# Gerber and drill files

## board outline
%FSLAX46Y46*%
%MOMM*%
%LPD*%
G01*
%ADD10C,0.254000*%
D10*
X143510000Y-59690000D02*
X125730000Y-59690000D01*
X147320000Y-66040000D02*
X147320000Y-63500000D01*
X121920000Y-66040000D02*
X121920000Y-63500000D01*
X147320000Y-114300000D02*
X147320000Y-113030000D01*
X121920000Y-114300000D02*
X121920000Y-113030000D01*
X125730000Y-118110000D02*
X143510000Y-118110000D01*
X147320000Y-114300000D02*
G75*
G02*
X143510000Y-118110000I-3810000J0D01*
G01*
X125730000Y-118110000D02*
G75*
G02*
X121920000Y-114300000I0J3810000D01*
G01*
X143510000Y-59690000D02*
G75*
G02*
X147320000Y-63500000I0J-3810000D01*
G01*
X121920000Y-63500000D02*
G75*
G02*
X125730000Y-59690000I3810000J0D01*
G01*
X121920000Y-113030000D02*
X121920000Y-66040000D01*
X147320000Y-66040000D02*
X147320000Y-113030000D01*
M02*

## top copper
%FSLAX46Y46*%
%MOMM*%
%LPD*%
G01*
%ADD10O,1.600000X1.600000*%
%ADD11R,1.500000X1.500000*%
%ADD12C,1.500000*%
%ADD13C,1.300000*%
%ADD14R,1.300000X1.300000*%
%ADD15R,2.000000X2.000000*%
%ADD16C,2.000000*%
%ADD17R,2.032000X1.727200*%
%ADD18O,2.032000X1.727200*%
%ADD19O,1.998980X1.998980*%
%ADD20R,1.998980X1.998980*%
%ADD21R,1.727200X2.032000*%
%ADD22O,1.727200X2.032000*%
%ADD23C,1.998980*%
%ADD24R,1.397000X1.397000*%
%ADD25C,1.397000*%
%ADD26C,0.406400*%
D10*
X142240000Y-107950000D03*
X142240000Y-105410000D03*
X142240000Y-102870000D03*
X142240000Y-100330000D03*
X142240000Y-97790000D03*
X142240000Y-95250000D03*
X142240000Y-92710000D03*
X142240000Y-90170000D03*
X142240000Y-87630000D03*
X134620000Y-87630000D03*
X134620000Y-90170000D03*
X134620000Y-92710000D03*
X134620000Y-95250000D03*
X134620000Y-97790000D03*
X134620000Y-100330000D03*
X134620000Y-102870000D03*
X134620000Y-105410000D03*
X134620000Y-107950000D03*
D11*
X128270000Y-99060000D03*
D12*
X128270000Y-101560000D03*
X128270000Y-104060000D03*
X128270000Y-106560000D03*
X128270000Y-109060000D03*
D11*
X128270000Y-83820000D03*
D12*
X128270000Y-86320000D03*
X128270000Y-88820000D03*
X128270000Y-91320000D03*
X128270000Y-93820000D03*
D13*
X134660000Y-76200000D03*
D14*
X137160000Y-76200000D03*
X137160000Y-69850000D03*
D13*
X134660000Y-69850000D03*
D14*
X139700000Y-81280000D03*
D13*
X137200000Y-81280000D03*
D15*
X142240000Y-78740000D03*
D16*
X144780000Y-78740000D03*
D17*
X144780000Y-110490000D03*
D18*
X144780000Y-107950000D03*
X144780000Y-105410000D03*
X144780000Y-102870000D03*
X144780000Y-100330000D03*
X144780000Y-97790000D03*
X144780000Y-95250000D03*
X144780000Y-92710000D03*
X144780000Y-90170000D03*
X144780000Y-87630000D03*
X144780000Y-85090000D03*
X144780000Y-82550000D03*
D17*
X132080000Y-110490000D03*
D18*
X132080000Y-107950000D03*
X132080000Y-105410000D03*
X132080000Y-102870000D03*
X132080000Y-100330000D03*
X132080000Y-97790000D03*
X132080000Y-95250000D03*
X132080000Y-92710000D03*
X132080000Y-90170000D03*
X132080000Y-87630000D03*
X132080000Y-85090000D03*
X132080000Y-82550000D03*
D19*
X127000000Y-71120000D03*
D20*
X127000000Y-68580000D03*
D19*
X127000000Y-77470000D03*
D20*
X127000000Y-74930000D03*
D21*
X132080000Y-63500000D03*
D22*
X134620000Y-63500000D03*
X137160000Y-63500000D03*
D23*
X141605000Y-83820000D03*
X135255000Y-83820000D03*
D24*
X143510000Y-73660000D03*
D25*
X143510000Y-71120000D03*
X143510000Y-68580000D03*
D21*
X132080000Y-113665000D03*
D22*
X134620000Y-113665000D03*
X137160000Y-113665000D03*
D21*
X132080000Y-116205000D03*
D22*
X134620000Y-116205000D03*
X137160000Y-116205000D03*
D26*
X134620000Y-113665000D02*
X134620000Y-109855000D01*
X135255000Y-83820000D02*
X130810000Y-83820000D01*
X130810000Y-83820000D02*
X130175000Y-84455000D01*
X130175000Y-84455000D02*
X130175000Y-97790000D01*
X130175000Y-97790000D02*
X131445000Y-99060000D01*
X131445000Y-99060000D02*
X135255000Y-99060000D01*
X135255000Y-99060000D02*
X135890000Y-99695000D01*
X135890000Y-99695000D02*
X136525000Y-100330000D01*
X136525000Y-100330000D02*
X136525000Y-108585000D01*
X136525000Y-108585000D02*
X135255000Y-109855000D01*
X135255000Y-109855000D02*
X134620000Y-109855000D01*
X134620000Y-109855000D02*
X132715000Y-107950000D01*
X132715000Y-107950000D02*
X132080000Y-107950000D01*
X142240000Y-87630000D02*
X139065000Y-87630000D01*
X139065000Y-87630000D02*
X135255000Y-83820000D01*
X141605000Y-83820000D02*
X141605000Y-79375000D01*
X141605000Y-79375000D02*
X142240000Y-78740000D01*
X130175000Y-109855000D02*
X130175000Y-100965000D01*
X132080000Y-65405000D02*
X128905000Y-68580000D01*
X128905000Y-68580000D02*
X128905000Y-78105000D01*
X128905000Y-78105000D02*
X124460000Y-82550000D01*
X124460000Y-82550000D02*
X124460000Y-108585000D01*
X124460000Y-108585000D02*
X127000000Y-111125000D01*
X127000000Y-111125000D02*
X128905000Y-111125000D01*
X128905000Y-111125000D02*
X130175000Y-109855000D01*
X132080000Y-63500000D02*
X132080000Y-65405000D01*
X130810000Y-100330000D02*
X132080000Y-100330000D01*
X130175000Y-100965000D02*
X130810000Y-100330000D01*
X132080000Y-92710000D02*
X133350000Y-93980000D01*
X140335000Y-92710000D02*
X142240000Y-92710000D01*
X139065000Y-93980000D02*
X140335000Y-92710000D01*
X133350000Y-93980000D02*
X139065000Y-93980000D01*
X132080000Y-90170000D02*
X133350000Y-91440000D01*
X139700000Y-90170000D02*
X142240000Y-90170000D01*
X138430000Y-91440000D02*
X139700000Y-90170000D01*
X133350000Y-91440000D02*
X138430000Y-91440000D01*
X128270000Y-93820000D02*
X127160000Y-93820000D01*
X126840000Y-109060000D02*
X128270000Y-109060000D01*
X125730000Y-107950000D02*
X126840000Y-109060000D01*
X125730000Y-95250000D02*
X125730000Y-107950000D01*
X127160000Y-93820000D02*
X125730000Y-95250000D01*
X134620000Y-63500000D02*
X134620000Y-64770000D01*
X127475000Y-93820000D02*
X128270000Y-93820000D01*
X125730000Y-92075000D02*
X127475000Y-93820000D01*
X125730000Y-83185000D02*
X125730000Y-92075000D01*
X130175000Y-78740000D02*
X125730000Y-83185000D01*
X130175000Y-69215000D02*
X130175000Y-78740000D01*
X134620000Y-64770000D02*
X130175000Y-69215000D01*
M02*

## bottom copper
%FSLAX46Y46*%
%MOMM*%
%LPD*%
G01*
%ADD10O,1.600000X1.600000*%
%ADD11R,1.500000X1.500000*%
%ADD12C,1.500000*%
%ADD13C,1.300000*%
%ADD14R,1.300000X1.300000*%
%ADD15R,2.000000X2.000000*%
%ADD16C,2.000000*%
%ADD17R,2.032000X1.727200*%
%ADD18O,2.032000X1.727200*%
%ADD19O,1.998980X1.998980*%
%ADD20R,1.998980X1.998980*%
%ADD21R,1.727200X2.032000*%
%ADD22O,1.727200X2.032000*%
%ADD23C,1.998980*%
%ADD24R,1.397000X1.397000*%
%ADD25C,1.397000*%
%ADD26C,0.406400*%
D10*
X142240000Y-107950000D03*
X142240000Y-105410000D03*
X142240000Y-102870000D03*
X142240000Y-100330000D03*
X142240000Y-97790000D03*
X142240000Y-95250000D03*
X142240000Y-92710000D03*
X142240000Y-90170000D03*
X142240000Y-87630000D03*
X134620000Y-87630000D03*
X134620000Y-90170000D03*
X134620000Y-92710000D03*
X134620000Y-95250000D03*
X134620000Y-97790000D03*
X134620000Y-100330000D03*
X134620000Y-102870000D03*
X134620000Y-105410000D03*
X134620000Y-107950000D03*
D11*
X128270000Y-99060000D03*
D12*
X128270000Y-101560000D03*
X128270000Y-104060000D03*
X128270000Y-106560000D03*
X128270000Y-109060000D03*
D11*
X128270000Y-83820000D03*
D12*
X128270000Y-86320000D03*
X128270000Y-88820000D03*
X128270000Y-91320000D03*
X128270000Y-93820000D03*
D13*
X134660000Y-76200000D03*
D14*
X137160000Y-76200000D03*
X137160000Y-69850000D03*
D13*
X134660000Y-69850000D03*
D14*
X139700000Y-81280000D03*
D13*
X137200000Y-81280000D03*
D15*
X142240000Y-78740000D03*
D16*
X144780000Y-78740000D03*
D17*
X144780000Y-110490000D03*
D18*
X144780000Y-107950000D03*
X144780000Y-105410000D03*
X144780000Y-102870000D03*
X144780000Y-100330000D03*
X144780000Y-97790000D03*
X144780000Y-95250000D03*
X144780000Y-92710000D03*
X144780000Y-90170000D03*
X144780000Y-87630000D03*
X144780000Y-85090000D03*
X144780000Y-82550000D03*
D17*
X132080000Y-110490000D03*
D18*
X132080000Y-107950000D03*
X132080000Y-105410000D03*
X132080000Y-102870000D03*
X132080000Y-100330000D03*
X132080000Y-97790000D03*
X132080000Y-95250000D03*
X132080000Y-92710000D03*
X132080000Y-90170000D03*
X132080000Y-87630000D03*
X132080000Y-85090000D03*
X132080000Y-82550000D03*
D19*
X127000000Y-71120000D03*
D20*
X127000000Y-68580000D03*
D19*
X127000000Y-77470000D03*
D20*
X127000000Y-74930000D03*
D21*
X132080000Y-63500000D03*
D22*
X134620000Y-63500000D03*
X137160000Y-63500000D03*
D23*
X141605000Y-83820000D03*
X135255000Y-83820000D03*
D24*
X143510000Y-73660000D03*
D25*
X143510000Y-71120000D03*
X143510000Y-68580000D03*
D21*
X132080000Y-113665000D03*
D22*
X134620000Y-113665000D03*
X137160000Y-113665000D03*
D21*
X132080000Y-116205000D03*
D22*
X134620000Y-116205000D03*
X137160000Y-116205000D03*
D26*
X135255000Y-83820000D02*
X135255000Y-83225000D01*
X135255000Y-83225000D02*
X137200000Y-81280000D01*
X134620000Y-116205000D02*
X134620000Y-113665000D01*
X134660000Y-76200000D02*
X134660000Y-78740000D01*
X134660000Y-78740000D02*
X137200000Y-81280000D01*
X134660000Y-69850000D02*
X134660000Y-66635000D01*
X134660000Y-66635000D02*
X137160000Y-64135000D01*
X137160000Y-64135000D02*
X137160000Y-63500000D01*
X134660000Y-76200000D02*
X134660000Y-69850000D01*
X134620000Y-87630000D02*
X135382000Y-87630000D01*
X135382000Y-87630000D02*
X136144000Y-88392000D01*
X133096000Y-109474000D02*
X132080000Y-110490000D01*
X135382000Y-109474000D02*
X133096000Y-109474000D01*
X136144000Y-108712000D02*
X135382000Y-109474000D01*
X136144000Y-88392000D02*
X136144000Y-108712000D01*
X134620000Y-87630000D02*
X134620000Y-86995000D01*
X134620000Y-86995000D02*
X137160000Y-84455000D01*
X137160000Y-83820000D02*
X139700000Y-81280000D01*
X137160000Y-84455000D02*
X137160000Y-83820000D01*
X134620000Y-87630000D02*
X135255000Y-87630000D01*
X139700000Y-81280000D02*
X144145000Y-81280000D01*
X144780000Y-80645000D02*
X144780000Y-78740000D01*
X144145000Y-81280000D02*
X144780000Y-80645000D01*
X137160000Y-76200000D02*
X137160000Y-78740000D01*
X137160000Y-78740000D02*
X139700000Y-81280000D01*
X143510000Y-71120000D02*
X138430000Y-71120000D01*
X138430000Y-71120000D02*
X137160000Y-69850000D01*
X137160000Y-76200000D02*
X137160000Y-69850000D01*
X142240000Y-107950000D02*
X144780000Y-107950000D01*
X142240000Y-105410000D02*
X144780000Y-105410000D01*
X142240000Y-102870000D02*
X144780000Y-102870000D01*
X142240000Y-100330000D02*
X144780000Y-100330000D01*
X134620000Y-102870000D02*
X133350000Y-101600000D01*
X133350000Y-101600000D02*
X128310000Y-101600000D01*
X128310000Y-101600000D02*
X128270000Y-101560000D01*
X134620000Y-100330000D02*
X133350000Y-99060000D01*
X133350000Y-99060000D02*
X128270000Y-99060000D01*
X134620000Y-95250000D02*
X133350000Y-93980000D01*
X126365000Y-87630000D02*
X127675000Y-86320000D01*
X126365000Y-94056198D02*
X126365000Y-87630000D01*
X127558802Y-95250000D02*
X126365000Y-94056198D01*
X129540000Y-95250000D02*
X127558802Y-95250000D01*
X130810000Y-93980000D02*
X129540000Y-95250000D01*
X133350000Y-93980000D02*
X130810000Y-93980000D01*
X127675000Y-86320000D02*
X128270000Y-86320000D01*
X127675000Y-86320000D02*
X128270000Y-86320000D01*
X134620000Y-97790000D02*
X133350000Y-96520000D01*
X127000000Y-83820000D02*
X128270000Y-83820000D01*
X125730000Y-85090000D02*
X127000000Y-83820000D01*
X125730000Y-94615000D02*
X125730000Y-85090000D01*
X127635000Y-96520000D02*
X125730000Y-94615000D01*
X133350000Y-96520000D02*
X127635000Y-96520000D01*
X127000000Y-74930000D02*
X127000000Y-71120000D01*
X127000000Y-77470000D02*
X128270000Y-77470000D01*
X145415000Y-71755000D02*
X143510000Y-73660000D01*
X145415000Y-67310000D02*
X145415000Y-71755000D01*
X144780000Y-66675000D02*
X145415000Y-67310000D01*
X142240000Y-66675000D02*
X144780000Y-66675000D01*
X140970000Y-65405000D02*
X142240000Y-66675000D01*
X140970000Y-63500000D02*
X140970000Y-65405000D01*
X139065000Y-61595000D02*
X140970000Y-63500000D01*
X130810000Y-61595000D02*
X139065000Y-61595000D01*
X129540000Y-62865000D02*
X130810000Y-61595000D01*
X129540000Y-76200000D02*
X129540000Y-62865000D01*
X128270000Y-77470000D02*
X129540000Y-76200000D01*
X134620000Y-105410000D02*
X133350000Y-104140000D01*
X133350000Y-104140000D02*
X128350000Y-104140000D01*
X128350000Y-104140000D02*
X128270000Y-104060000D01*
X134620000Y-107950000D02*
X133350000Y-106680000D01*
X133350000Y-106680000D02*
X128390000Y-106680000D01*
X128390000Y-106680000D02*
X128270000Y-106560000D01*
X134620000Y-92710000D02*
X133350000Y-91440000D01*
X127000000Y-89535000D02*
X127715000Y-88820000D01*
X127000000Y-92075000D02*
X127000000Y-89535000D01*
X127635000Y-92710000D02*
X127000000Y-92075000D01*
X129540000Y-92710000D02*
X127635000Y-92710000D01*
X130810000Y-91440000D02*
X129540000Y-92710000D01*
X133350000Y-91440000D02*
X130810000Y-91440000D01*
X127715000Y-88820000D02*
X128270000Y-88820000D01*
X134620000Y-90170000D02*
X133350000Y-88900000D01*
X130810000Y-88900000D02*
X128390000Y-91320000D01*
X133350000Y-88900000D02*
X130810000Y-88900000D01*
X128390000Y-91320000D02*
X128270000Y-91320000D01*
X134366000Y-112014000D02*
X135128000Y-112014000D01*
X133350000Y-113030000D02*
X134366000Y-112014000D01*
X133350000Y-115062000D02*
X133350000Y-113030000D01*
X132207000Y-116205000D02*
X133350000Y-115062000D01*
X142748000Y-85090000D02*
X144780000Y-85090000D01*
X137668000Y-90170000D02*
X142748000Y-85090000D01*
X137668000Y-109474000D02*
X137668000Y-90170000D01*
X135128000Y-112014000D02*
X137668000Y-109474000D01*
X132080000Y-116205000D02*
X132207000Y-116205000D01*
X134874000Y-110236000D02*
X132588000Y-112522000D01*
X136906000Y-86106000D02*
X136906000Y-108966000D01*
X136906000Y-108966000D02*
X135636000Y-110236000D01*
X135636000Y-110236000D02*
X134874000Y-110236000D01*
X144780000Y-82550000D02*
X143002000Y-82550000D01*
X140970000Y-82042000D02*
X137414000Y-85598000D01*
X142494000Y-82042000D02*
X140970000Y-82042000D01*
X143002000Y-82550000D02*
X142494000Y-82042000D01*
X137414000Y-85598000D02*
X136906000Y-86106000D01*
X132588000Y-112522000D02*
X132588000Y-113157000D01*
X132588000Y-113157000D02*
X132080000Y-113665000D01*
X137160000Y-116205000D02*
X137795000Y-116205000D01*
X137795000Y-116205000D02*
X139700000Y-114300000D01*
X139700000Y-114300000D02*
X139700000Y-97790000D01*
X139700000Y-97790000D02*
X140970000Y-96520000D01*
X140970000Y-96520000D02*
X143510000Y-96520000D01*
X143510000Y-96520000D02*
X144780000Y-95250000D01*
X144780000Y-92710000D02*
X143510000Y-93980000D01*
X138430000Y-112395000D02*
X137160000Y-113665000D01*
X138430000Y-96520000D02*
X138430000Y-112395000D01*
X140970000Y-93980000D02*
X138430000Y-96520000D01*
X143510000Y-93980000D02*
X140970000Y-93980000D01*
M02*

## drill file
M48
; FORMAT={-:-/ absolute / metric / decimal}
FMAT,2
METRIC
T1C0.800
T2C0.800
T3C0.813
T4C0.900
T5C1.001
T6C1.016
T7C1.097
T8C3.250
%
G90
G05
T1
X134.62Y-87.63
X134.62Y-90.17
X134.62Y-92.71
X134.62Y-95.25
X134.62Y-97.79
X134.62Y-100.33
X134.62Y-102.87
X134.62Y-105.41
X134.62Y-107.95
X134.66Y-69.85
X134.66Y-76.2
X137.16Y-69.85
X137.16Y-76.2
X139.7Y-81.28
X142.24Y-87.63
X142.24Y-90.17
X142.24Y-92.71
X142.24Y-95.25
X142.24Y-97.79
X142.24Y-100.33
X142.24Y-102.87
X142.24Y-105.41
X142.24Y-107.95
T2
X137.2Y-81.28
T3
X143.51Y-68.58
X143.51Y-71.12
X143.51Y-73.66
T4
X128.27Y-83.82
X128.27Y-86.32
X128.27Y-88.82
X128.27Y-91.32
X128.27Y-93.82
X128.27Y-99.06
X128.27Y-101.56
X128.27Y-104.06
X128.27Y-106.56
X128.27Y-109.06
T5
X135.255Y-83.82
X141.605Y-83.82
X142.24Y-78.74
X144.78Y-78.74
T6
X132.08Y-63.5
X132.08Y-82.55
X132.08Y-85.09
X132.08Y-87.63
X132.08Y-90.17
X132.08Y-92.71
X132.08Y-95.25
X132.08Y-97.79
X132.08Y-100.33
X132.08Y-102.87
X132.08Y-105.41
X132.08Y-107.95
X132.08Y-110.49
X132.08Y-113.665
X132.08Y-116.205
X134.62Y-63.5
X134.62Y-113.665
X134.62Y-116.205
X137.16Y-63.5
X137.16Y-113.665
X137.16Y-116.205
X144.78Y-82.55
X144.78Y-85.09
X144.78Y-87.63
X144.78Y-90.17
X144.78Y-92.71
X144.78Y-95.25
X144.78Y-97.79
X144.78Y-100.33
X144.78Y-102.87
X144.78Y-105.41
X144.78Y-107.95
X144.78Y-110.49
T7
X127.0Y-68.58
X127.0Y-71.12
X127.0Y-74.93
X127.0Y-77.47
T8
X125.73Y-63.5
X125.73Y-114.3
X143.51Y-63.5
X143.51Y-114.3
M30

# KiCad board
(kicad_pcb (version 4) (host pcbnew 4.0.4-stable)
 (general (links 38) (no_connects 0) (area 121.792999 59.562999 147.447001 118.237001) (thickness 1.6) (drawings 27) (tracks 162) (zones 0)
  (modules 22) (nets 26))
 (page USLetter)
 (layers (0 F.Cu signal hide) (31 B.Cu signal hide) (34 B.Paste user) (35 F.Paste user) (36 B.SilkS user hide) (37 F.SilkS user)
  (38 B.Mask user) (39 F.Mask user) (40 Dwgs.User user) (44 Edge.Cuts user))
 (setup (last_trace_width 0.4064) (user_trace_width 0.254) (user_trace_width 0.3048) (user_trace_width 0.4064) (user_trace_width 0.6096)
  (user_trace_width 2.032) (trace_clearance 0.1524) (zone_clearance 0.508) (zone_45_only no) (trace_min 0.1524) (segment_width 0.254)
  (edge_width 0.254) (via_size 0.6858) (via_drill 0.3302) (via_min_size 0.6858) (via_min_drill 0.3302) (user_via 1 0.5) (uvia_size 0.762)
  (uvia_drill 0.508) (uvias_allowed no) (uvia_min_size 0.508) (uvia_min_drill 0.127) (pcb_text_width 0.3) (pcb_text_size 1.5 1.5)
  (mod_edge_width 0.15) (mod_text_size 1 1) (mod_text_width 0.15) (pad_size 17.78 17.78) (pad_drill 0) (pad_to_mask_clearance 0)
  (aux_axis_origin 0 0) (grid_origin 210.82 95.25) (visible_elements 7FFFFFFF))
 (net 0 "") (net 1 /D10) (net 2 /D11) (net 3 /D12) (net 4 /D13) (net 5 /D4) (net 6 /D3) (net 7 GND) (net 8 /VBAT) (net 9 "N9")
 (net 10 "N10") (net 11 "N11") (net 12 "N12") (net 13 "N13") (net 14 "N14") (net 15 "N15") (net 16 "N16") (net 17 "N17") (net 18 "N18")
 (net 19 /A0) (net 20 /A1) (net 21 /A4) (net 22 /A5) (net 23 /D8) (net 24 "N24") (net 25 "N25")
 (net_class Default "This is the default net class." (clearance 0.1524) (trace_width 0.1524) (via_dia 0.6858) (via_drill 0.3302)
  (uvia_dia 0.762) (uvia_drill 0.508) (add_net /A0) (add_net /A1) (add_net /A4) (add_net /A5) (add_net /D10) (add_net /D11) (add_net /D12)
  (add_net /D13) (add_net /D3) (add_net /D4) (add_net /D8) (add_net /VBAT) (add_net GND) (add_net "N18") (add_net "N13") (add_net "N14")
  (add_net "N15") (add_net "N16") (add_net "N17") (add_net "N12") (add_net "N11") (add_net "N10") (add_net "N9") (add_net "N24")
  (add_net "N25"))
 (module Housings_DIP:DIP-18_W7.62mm (layer F.Cu) (at 142.24 107.95 180)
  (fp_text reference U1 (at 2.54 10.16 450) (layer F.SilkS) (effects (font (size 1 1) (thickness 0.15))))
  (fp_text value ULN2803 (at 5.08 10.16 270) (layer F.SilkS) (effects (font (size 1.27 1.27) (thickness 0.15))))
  (pad 1 thru_hole oval (at 0 0 180) (size 1.6 1.6) (drill 0.8) (layers *.Cu *.Mask F.SilkS) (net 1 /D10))
  (pad 2 thru_hole oval (at 0 2.54 180) (size 1.6 1.6) (drill 0.8) (layers *.Cu *.Mask F.SilkS) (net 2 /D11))
  (pad 3 thru_hole oval (at 0 5.08 180) (size 1.6 1.6) (drill 0.8) (layers *.Cu *.Mask F.SilkS) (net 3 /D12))
  (pad 4 thru_hole oval (at 0 7.62 180) (size 1.6 1.6) (drill 0.8) (layers *.Cu *.Mask F.SilkS) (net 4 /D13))
  (pad 5 thru_hole oval (at 0 10.16 180) (size 1.6 1.6) (drill 0.8) (layers *.Cu *.Mask F.SilkS))
  (pad 6 thru_hole oval (at 0 12.7 180) (size 1.6 1.6) (drill 0.8) (layers *.Cu *.Mask F.SilkS))
  (pad 7 thru_hole oval (at 0 15.24 180) (size 1.6 1.6) (drill 0.8) (layers *.Cu *.Mask F.SilkS) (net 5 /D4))
  (pad 8 thru_hole oval (at 0 17.78 180) (size 1.6 1.6) (drill 0.8) (layers *.Cu *.Mask F.SilkS) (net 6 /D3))
  (pad 9 thru_hole oval (at 0 20.32 180) (size 1.6 1.6) (drill 0.8) (layers *.Cu *.Mask F.SilkS) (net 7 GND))
  (pad 10 thru_hole oval (at 7.62 20.32 180) (size 1.6 1.6) (drill 0.8) (layers *.Cu *.Mask F.SilkS) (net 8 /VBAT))
  (pad 11 thru_hole oval (at 7.62 17.78 180) (size 1.6 1.6) (drill 0.8) (layers *.Cu *.Mask F.SilkS) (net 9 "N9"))
  (pad 12 thru_hole oval (at 7.62 15.24 180) (size 1.6 1.6) (drill 0.8) (layers *.Cu *.Mask F.SilkS) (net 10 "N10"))
  (pad 13 thru_hole oval (at 7.62 12.7 180) (size 1.6 1.6) (drill 0.8) (layers *.Cu *.Mask F.SilkS) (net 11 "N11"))
  (pad 14 thru_hole oval (at 7.62 10.16 180) (size 1.6 1.6) (drill 0.8) (layers *.Cu *.Mask F.SilkS) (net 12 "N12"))
  (pad 15 thru_hole oval (at 7.62 7.62 180) (size 1.6 1.6) (drill 0.8) (layers *.Cu *.Mask F.SilkS) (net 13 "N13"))
  (pad 16 thru_hole oval (at 7.62 5.08 180) (size 1.6 1.6) (drill 0.8) (layers *.Cu *.Mask F.SilkS) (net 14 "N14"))
  (pad 17 thru_hole oval (at 7.62 2.54 180) (size 1.6 1.6) (drill 0.8) (layers *.Cu *.Mask F.SilkS) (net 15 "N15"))
  (pad 18 thru_hole oval (at 7.62 0 180) (size 1.6 1.6) (drill 0.8) (layers *.Cu *.Mask F.SilkS) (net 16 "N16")))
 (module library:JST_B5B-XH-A (layer F.Cu) (at 128.27 99.06 270)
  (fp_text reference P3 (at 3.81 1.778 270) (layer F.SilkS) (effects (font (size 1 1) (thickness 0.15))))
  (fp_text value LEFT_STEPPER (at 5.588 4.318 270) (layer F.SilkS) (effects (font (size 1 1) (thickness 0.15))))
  (pad 1 thru_hole rect (at 0 0 270) (size 1.5 1.5) (drill 0.9) (layers *.Cu *.Mask F.SilkS) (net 13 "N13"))
  (pad 2 thru_hole circle (at 2.5 0 270) (size 1.5 1.5) (drill 0.9) (layers *.Cu *.Mask F.SilkS) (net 14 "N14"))
  (pad 3 thru_hole circle (at 5 0 270) (size 1.5 1.5) (drill 0.9) (layers *.Cu *.Mask F.SilkS) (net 15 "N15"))
  (pad 4 thru_hole circle (at 7.5 0 270) (size 1.5 1.5) (drill 0.9) (layers *.Cu *.Mask F.SilkS) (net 16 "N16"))
  (pad 5 thru_hole circle (at 10 0 270) (size 1.5 1.5) (drill 0.9) (layers *.Cu *.Mask F.SilkS) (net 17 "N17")))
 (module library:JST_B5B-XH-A (layer F.Cu) (at 128.27 83.82 270)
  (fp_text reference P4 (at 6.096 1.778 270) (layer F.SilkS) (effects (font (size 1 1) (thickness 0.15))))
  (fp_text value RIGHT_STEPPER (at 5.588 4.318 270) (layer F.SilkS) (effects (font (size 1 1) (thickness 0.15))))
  (pad 1 thru_hole rect (at 0 0 270) (size 1.5 1.5) (drill 0.9) (layers *.Cu *.Mask F.SilkS) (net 12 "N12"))
  (pad 2 thru_hole circle (at 2.5 0 270) (size 1.5 1.5) (drill 0.9) (layers *.Cu *.Mask F.SilkS) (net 11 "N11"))
  (pad 3 thru_hole circle (at 5 0 270) (size 1.5 1.5) (drill 0.9) (layers *.Cu *.Mask F.SilkS) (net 10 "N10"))
  (pad 4 thru_hole circle (at 7.5 0 270) (size 1.5 1.5) (drill 0.9) (layers *.Cu *.Mask F.SilkS) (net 9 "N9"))
  (pad 5 thru_hole circle (at 10 0 270) (size 1.5 1.5) (drill 0.9) (layers *.Cu *.Mask F.SilkS) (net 17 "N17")))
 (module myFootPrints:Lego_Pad (layer F.Cu) (at 125.73 114.3)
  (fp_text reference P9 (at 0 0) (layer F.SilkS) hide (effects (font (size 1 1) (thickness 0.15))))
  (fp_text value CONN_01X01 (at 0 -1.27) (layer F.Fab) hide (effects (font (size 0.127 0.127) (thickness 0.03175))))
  (pad "" np_thru_hole circle (at 0 0) (size 3.25 3.25) (drill 3.25) (layers *.Cu *.Mask)))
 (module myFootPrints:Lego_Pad (layer F.Cu) (at 143.51 114.3)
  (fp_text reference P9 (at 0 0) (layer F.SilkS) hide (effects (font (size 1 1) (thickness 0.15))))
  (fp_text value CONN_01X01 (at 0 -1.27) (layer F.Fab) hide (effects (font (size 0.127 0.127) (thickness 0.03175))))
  (pad "" np_thru_hole circle (at 0 0) (size 3.25 3.25) (drill 3.25) (layers *.Cu *.Mask)))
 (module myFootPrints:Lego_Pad (layer F.Cu) (at 143.51 63.5)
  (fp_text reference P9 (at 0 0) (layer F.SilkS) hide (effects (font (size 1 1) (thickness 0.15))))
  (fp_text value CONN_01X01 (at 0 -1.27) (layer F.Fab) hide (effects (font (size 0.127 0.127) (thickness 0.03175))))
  (pad "" np_thru_hole circle (at 0 0) (size 3.25 3.25) (drill 3.25) (layers *.Cu *.Mask)))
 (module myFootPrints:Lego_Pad (layer F.Cu) (at 125.73 63.5)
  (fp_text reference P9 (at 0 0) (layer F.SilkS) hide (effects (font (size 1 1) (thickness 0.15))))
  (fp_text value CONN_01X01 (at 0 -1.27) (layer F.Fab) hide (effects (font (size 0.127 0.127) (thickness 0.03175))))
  (pad "" np_thru_hole circle (at 0 0) (size 3.25 3.25) (drill 3.25) (layers *.Cu *.Mask)))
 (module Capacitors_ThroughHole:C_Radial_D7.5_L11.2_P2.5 (layer F.Cu) (at 137.16 76.2 180)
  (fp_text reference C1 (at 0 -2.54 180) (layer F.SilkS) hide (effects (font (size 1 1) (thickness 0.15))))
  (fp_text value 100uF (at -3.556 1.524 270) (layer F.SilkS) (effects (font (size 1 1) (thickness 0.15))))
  (pad 2 thru_hole circle (at 2.5 0 180) (size 1.3 1.3) (drill 0.8) (layers *.Cu *.Mask F.SilkS) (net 7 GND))
  (pad 1 thru_hole rect (at 0 0 180) (size 1.3 1.3) (drill 0.8) (layers *.Cu *.Mask F.SilkS) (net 8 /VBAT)))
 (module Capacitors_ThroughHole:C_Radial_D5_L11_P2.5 (layer F.Cu) (at 137.16 69.85 180)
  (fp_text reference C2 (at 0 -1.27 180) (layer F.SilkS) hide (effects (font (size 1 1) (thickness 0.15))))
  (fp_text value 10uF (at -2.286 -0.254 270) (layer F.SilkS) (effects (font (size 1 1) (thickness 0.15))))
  (pad 1 thru_hole rect (at 0 0 180) (size 1.3 1.3) (drill 0.8) (layers *.Cu *.Mask F.SilkS) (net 8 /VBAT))
  (pad 2 thru_hole circle (at 2.5 0 180) (size 1.3 1.3) (drill 0.8) (layers *.Cu *.Mask F.SilkS) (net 7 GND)))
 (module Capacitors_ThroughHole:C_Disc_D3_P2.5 (layer F.Cu) (at 139.7 81.28 180)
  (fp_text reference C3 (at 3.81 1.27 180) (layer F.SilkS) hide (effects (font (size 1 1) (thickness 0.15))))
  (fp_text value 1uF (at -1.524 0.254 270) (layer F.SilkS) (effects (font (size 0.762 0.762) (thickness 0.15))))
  (pad 1 thru_hole rect (at 0 0 180) (size 1.3 1.3) (drill 0.8) (layers *.Cu *.Mask F.SilkS) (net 8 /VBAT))
  (pad 2 thru_hole circle (at 2.5 0 180) (size 1.3 1.3) (drill 0.8001) (layers *.Cu *.Mask F.SilkS) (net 7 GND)))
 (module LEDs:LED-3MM (layer F.Cu) (at 142.24 78.74)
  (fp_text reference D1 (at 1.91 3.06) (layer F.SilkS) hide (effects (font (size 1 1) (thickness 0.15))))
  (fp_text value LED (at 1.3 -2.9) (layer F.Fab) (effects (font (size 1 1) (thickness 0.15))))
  (pad 1 thru_hole rect (at 0 0 90) (size 2 2) (drill 1.00076) (layers *.Cu *.Mask F.SilkS) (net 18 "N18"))
  (pad 2 thru_hole circle (at 2.54 0) (size 2 2) (drill 1.00076) (layers *.Cu *.Mask F.SilkS) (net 8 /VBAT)))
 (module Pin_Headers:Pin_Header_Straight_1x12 (layer F.Cu) (at 144.78 110.49 180)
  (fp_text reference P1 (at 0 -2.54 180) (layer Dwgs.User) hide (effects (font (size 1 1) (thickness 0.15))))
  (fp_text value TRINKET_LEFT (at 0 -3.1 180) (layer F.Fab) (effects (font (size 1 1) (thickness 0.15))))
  (pad 1 thru_hole rect (at 0 0 180) (size 2.032 1.7272) (drill 1.016) (layers *.Cu *.Mask F.SilkS))
  (pad 2 thru_hole oval (at 0 2.54 180) (size 2.032 1.7272) (drill 1.016) (layers *.Cu *.Mask F.SilkS) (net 1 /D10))
  (pad 3 thru_hole oval (at 0 5.08 180) (size 2.032 1.7272) (drill 1.016) (layers *.Cu *.Mask F.SilkS) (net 2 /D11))
  (pad 4 thru_hole oval (at 0 7.62 180) (size 2.032 1.7272) (drill 1.016) (layers *.Cu *.Mask F.SilkS) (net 3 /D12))
  (pad 5 thru_hole oval (at 0 10.16 180) (size 2.032 1.7272) (drill 1.016) (layers *.Cu *.Mask F.SilkS) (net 4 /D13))
  (pad 6 thru_hole oval (at 0 12.7 180) (size 2.032 1.7272) (drill 1.016) (layers *.Cu *.Mask F.SilkS))
  (pad 7 thru_hole oval (at 0 15.24 180) (size 2.032 1.7272) (drill 1.016) (layers *.Cu *.Mask F.SilkS) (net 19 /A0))
  (pad 8 thru_hole oval (at 0 17.78 180) (size 2.032 1.7272) (drill 1.016) (layers *.Cu *.Mask F.SilkS) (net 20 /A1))
  (pad 9 thru_hole oval (at 0 20.32 180) (size 2.032 1.7272) (drill 1.016) (layers *.Cu *.Mask F.SilkS))
  (pad 10 thru_hole oval (at 0 22.86 180) (size 2.032 1.7272) (drill 1.016) (layers *.Cu *.Mask F.SilkS))
  (pad 11 thru_hole oval (at 0 25.4 180) (size 2.032 1.7272) (drill 1.016) (layers *.Cu *.Mask F.SilkS) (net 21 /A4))
  (pad 12 thru_hole oval (at 0 27.94 180) (size 2.032 1.7272) (drill 1.016) (layers *.Cu *.Mask F.SilkS) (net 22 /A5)))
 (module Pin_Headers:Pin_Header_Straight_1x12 (layer F.Cu) (at 132.08 110.49 180)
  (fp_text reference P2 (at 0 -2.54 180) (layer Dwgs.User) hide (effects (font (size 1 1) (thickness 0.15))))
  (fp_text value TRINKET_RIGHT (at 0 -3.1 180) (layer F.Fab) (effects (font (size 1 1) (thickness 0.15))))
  (pad 1 thru_hole rect (at 0 0 180) (size 2.032 1.7272) (drill 1.016) (layers *.Cu *.Mask F.SilkS) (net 8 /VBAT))
  (pad 2 thru_hole oval (at 0 2.54 180) (size 2.032 1.7272) (drill 1.016) (layers *.Cu *.Mask F.SilkS) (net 7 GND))
  (pad 3 thru_hole oval (at 0 5.08 180) (size 2.032 1.7272) (drill 1.016) (layers *.Cu *.Mask F.SilkS))
  (pad 4 thru_hole oval (at 0 7.62 180) (size 2.032 1.7272) (drill 1.016) (layers *.Cu *.Mask F.SilkS))
  (pad 5 thru_hole oval (at 0 10.16 180) (size 2.032 1.7272) (drill 1.016) (layers *.Cu *.Mask F.SilkS) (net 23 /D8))
  (pad 6 thru_hole oval (at 0 12.7 180) (size 2.032 1.7272) (drill 1.016) (layers *.Cu *.Mask F.SilkS))
  (pad 7 thru_hole oval (at 0 15.24 180) (size 2.032 1.7272) (drill 1.016) (layers *.Cu *.Mask F.SilkS))
  (pad 8 thru_hole oval (at 0 17.78 180) (size 2.032 1.7272) (drill 1.016) (layers *.Cu *.Mask F.SilkS) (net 5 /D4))
  (pad 9 thru_hole oval (at 0 20.32 180) (size 2.032 1.7272) (drill 1.016) (layers *.Cu *.Mask F.SilkS) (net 6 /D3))
  (pad 10 thru_hole oval (at 0 22.86 180) (size 2.032 1.7272) (drill 1.016) (layers *.Cu *.Mask F.SilkS))
  (pad 11 thru_hole oval (at 0 25.4 180) (size 2.032 1.7272) (drill 1.016) (layers *.Cu *.Mask F.SilkS))
  (pad 12 thru_hole oval (at 0 27.94 180) (size 2.032 1.7272) (drill 1.016) (layers *.Cu *.Mask F.SilkS)))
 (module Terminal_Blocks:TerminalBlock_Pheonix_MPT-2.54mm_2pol (layer F.Cu) (at 127 68.58 270)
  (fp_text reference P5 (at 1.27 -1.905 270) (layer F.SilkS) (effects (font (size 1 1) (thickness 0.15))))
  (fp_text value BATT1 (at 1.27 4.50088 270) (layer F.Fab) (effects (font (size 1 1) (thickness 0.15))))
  (pad 2 thru_hole oval (at 2.54 0 270) (size 1.99898 1.99898) (drill 1.09728) (layers *.Cu *.Mask F.SilkS) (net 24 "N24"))
  (pad 1 thru_hole rect (at 0 0 270) (size 1.99898 1.99898) (drill 1.09728) (layers *.Cu *.Mask F.SilkS)))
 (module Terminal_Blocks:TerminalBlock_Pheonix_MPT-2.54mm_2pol (layer F.Cu) (at 127 74.93 270)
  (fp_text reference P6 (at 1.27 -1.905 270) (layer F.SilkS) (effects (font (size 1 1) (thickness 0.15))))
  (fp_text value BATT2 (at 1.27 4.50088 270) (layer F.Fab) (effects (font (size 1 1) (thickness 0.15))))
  (pad 2 thru_hole oval (at 2.54 0 270) (size 1.99898 1.99898) (drill 1.09728) (layers *.Cu *.Mask F.SilkS) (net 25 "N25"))
  (pad 1 thru_hole rect (at 0 0 270) (size 1.99898 1.99898) (drill 1.09728) (layers *.Cu *.Mask F.SilkS) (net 24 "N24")))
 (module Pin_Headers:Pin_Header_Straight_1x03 (layer F.Cu) (at 132.08 63.5 90)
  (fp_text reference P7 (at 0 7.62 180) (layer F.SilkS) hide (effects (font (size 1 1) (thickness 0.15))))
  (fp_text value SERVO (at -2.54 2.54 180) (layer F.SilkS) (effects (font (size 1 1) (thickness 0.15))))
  (pad 1 thru_hole rect (at 0 0 90) (size 2.032 1.7272) (drill 1.016) (layers *.Cu *.Mask F.SilkS) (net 23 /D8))
  (pad 2 thru_hole oval (at 0 2.54 90) (size 2.032 1.7272) (drill 1.016) (layers *.Cu *.Mask F.SilkS) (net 17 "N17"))
  (pad 3 thru_hole oval (at 0 5.08 90) (size 2.032 1.7272) (drill 1.016) (layers *.Cu *.Mask F.SilkS) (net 7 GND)))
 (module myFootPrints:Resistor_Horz (layer F.Cu) (at 138.43 83.82 180)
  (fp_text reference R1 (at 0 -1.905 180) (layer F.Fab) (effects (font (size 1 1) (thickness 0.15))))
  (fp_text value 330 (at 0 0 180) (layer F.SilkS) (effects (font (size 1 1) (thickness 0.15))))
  (pad 1 thru_hole circle (at -3.175 0 180) (size 1.99898 1.99898) (drill 1.00076) (layers *.Cu *.SilkS *.Mask) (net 18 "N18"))
  (pad 2 thru_hole circle (at 3.175 0 180) (size 1.99898 1.99898) (drill 1.00076) (layers *.Cu *.SilkS *.Mask) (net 7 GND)))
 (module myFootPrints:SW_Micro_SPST (layer F.Cu) (at 143.51 71.12 90)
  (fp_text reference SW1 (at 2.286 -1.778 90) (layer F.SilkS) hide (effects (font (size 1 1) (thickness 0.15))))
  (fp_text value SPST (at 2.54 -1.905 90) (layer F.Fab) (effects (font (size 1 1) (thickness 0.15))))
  (pad 1 thru_hole rect (at -2.54 0 90) (size 1.397 1.397) (drill 0.8128) (layers *.Cu *.Mask F.SilkS) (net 25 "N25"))
  (pad 2 thru_hole circle (at 0 0 90) (size 1.397 1.397) (drill 0.8128) (layers *.Cu *.Mask F.SilkS) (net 8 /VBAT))
  (pad 3 thru_hole circle (at 2.54 0 90) (size 1.397 1.397) (drill 0.8128) (layers *.Cu *.Mask F.SilkS)))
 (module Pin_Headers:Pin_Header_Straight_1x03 (layer F.Cu) (at 132.08 113.665 90)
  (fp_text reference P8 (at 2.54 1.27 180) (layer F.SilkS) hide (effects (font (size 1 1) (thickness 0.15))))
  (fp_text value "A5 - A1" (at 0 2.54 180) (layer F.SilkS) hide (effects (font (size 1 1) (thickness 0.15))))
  (pad 1 thru_hole rect (at 0 0 90) (size 2.032 1.7272) (drill 1.016) (layers *.Cu *.Mask F.SilkS) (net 22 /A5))
  (pad 2 thru_hole oval (at 0 2.54 90) (size 2.032 1.7272) (drill 1.016) (layers *.Cu *.Mask F.SilkS) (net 7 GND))
  (pad 3 thru_hole oval (at 0 5.08 90) (size 2.032 1.7272) (drill 1.016) (layers *.Cu *.Mask F.SilkS) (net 20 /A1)))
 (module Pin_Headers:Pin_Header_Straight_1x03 (layer F.Cu) (at 132.08 116.205 90)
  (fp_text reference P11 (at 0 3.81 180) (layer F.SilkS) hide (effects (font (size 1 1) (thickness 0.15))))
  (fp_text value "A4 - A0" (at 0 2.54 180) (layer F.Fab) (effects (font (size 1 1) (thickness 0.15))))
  (pad 1 thru_hole rect (at 0 0 90) (size 2.032 1.7272) (drill 1.016) (layers *.Cu *.Mask F.SilkS) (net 21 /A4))
  (pad 2 thru_hole oval (at 0 2.54 90) (size 2.032 1.7272) (drill 1.016) (layers *.Cu *.Mask F.SilkS) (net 7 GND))
  (pad 3 thru_hole oval (at 0 5.08 90) (size 2.032 1.7272) (drill 1.016) (layers *.Cu *.Mask F.SilkS) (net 19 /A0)))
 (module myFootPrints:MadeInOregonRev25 (layer F.Cu) (at 138.43 102.235 90)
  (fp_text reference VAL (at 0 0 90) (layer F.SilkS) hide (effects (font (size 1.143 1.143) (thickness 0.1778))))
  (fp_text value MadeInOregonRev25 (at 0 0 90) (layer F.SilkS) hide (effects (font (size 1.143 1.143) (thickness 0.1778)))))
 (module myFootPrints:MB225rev (layer F.Cu) (at 138.43 109.22 90)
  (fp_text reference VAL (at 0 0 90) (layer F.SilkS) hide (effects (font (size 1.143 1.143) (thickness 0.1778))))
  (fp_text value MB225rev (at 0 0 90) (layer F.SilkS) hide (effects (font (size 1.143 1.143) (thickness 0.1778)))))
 (gr_line (start 143.51 59.69) (end 125.73 59.69) (angle 90) (layer Edge.Cuts) (width 0.254))
 (gr_line (start 147.32 66.04) (end 147.32 63.5) (angle 90) (layer Edge.Cuts) (width 0.254))
 (gr_line (start 121.92 66.04) (end 121.92 63.5) (angle 90) (layer Edge.Cuts) (width 0.254))
 (gr_line (start 147.32 114.3) (end 147.32 113.03) (angle 90) (layer Edge.Cuts) (width 0.254))
 (gr_line (start 121.92 114.3) (end 121.92 113.03) (angle 90) (layer Edge.Cuts) (width 0.254))
 (gr_line (start 125.73 118.11) (end 143.51 118.11) (angle 90) (layer Edge.Cuts) (width 0.254))
 (gr_arc (start 143.51 114.3) (end 147.32 114.3) (angle 90) (layer Edge.Cuts) (width 0.254))
 (gr_arc (start 125.73 114.3) (end 125.73 118.11) (angle 90) (layer Edge.Cuts) (width 0.254))
 (gr_arc (start 143.51 63.5) (end 143.51 59.69) (angle 90) (layer Edge.Cuts) (width 0.254))
 (gr_arc (start 125.73 63.5) (end 121.92 63.5) (angle 90) (layer Edge.Cuts) (width 0.254))
 (gr_line (start 121.92 113.03) (end 121.92 66.04) (angle 90) (layer Edge.Cuts) (width 0.254))
 (gr_line (start 147.32 66.04) (end 147.32 113.03) (angle 90) (layer Edge.Cuts) (width 0.254))
 (segment (start 134.62 113.665) (end 134.62 109.855) (width 0.4064) (layer F.Cu) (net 7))
 (segment (start 135.255 83.82) (end 130.81 83.82) (width 0.4064) (layer F.Cu) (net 7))
 (segment (start 130.81 83.82) (end 130.175 84.455) (width 0.4064) (layer F.Cu) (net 7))
 (segment (start 130.175 84.455) (end 130.175 97.79) (width 0.4064) (layer F.Cu) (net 7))
 (segment (start 130.175 97.79) (end 131.445 99.06) (width 0.4064) (layer F.Cu) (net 7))
 (segment (start 131.445 99.06) (end 135.255 99.06) (width 0.4064) (layer F.Cu) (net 7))
 (segment (start 135.255 99.06) (end 135.89 99.695) (width 0.4064) (layer F.Cu) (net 7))
 (segment (start 135.89 99.695) (end 136.525 100.33) (width 0.4064) (layer F.Cu) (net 7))
 (segment (start 136.525 100.33) (end 136.525 108.585) (width 0.4064) (layer F.Cu) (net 7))
 (segment (start 136.525 108.585) (end 135.255 109.855) (width 0.4064) (layer F.Cu) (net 7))
 (segment (start 135.255 109.855) (end 134.62 109.855) (width 0.4064) (layer F.Cu) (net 7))
 (segment (start 134.62 109.855) (end 132.715 107.95) (width 0.4064) (layer F.Cu) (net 7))
 (segment (start 132.715 107.95) (end 132.08 107.95) (width 0.4064) (layer F.Cu) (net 7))
 (segment (start 142.24 87.63) (end 139.065 87.63) (width 0.4064) (layer F.Cu) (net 7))
 (segment (start 139.065 87.63) (end 135.255 83.82) (width 0.4064) (layer F.Cu) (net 7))
 (segment (start 135.255 83.82) (end 135.255 83.225) (width 0.4064) (layer B.Cu) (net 7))
 (segment (start 135.255 83.225) (end 137.2 81.28) (width 0.4064) (layer B.Cu) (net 7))
 (segment (start 134.62 116.205) (end 134.62 113.665) (width 0.4064) (layer B.Cu) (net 7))
 (segment (start 134.66 76.2) (end 134.66 78.74) (width 0.4064) (layer B.Cu) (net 7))
 (segment (start 134.66 78.74) (end 137.2 81.28) (width 0.4064) (layer B.Cu) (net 7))
 (segment (start 134.66 69.85) (end 134.66 66.635) (width 0.4064) (layer B.Cu) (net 7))
 (segment (start 134.66 66.635) (end 137.16 64.135) (width 0.4064) (layer B.Cu) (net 7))
 (segment (start 137.16 64.135) (end 137.16 63.5) (width 0.4064) (layer B.Cu) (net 7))
 (segment (start 134.66 76.2) (end 134.66 69.85) (width 0.4064) (layer B.Cu) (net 7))
 (segment (start 141.605 83.82) (end 141.605 79.375) (width 0.4064) (layer F.Cu) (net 18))
 (segment (start 141.605 79.375) (end 142.24 78.74) (width 0.4064) (layer F.Cu) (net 18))
 (segment (start 134.62 87.63) (end 135.382 87.63) (width 0.4064) (layer B.Cu) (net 8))
 (segment (start 135.382 87.63) (end 136.144 88.392) (width 0.4064) (layer B.Cu) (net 8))
 (segment (start 133.096 109.474) (end 132.08 110.49) (width 0.4064) (layer B.Cu) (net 8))
 (segment (start 135.382 109.474) (end 133.096 109.474) (width 0.4064) (layer B.Cu) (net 8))
 (segment (start 136.144 108.712) (end 135.382 109.474) (width 0.4064) (layer B.Cu) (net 8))
 (segment (start 136.144 88.392) (end 136.144 108.712) (width 0.4064) (layer B.Cu) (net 8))
 (segment (start 134.62 87.63) (end 134.62 86.995) (width 0.4064) (layer B.Cu) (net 8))
 (segment (start 134.62 86.995) (end 137.16 84.455) (width 0.4064) (layer B.Cu) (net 8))
 (segment (start 137.16 83.82) (end 139.7 81.28) (width 0.4064) (layer B.Cu) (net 8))
 (segment (start 137.16 84.455) (end 137.16 83.82) (width 0.4064) (layer B.Cu) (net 8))
 (segment (start 134.62 87.63) (end 135.255 87.63) (width 0.4064) (layer B.Cu) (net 8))
 (segment (start 139.7 81.28) (end 144.145 81.28) (width 0.4064) (layer B.Cu) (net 8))
 (segment (start 144.78 80.645) (end 144.78 78.74) (width 0.4064) (layer B.Cu) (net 8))
 (segment (start 144.145 81.28) (end 144.78 80.645) (width 0.4064) (layer B.Cu) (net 8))
 (segment (start 137.16 76.2) (end 137.16 78.74) (width 0.4064) (layer B.Cu) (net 8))
 (segment (start 137.16 78.74) (end 139.7 81.28) (width 0.4064) (layer B.Cu) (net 8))
 (segment (start 143.51 71.12) (end 138.43 71.12) (width 0.4064) (layer B.Cu) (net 8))
 (segment (start 138.43 71.12) (end 137.16 69.85) (width 0.4064) (layer B.Cu) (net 8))
 (segment (start 137.16 76.2) (end 137.16 69.85) (width 0.4064) (layer B.Cu) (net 8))
 (segment (start 142.24 107.95) (end 144.78 107.95) (width 0.4064) (layer B.Cu) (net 1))
 (segment (start 142.24 105.41) (end 144.78 105.41) (width 0.4064) (layer B.Cu) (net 2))
 (segment (start 142.24 102.87) (end 144.78 102.87) (width 0.4064) (layer B.Cu) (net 3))
 (segment (start 142.24 100.33) (end 144.78 100.33) (width 0.4064) (layer B.Cu) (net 4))
 (segment (start 130.175 109.855) (end 130.175 100.965) (width 0.4064) (layer F.Cu) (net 23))
 (segment (start 132.08 65.405) (end 128.905 68.58) (width 0.4064) (layer F.Cu) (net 23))
 (segment (start 128.905 68.58) (end 128.905 78.105) (width 0.4064) (layer F.Cu) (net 23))
 (segment (start 128.905 78.105) (end 124.46 82.55) (width 0.4064) (layer F.Cu) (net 23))
 (segment (start 124.46 82.55) (end 124.46 108.585) (width 0.4064) (layer F.Cu) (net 23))
 (segment (start 124.46 108.585) (end 127 111.125) (width 0.4064) (layer F.Cu) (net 23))
 (segment (start 127 111.125) (end 128.905 111.125) (width 0.4064) (layer F.Cu) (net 23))
 (segment (start 128.905 111.125) (end 130.175 109.855) (width 0.4064) (layer F.Cu) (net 23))
 (segment (start 132.08 63.5) (end 132.08 65.405) (width 0.4064) (layer F.Cu) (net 23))
 (segment (start 130.81 100.33) (end 132.08 100.33) (width 0.4064) (layer F.Cu) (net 23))
 (segment (start 130.175 100.965) (end 130.81 100.33) (width 0.4064) (layer F.Cu) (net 23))
 (segment (start 132.08 92.71) (end 133.35 93.98) (width 0.4064) (layer F.Cu) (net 5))
 (segment (start 140.335 92.71) (end 142.24 92.71) (width 0.4064) (layer F.Cu) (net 5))
 (segment (start 139.065 93.98) (end 140.335 92.71) (width 0.4064) (layer F.Cu) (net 5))
 (segment (start 133.35 93.98) (end 139.065 93.98) (width 0.4064) (layer F.Cu) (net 5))
 (segment (start 132.08 90.17) (end 133.35 91.44) (width 0.4064) (layer F.Cu) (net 6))
 (segment (start 139.7 90.17) (end 142.24 90.17) (width 0.4064) (layer F.Cu) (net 6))
 (segment (start 138.43 91.44) (end 139.7 90.17) (width 0.4064) (layer F.Cu) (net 6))
 (segment (start 133.35 91.44) (end 138.43 91.44) (width 0.4064) (layer F.Cu) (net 6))
 (segment (start 134.62 102.87) (end 133.35 101.6) (width 0.4064) (layer B.Cu) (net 14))
 (segment (start 133.35 101.6) (end 128.31 101.6) (width 0.4064) (layer B.Cu) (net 14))
 (segment (start 128.31 101.6) (end 128.27 101.56) (width 0.4064) (layer B.Cu) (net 14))
 (segment (start 134.62 100.33) (end 133.35 99.06) (width 0.4064) (layer B.Cu) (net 13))
 (segment (start 133.35 99.06) (end 128.27 99.06) (width 0.4064) (layer B.Cu) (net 13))
 (segment (start 134.62 95.25) (end 133.35 93.98) (width 0.4064) (layer B.Cu) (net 11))
 (segment (start 126.365 87.63) (end 127.675 86.32) (width 0.4064) (layer B.Cu) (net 11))
 (segment (start 126.365 94.056198) (end 126.365 87.63) (width 0.4064) (layer B.Cu) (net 11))
 (segment (start 127.558802 95.25) (end 126.365 94.056198) (width 0.4064) (layer B.Cu) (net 11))
 (segment (start 129.54 95.25) (end 127.558802 95.25) (width 0.4064) (layer B.Cu) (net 11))
 (segment (start 130.81 93.98) (end 129.54 95.25) (width 0.4064) (layer B.Cu) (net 11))
 (segment (start 133.35 93.98) (end 130.81 93.98) (width 0.4064) (layer B.Cu) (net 11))
 (segment (start 127.675 86.32) (end 128.27 86.32) (width 0.4064) (layer B.Cu) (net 11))
 (segment (start 127.675 86.32) (end 128.27 86.32) (width 0.4064) (layer B.Cu) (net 11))
 (segment (start 134.62 97.79) (end 133.35 96.52) (width 0.4064) (layer B.Cu) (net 12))
 (segment (start 127 83.82) (end 128.27 83.82) (width 0.4064) (layer B.Cu) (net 12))
 (segment (start 125.73 85.09) (end 127 83.82) (width 0.4064) (layer B.Cu) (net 12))
 (segment (start 125.73 94.615) (end 125.73 85.09) (width 0.4064) (layer B.Cu) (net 12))
 (segment (start 127.635 96.52) (end 125.73 94.615) (width 0.4064) (layer B.Cu) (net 12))
 (segment (start 133.35 96.52) (end 127.635 96.52) (width 0.4064) (layer B.Cu) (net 12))
 (segment (start 127 74.93) (end 127 71.12) (width 0.4064) (layer B.Cu) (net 24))
 (segment (start 127 77.47) (end 128.27 77.47) (width 0.4064) (layer B.Cu) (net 25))
 (segment (start 145.415 71.755) (end 143.51 73.66) (width 0.4064) (layer B.Cu) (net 25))
 (segment (start 145.415 67.31) (end 145.415 71.755) (width 0.4064) (layer B.Cu) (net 25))
 (segment (start 144.78 66.675) (end 145.415 67.31) (width 0.4064) (layer B.Cu) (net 25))
 (segment (start 142.24 66.675) (end 144.78 66.675) (width 0.4064) (layer B.Cu) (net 25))
 (segment (start 140.97 65.405) (end 142.24 66.675) (width 0.4064) (layer B.Cu) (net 25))
 (segment (start 140.97 63.5) (end 140.97 65.405) (width 0.4064) (layer B.Cu) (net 25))
 (segment (start 139.065 61.595) (end 140.97 63.5) (width 0.4064) (layer B.Cu) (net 25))
 (segment (start 130.81 61.595) (end 139.065 61.595) (width 0.4064) (layer B.Cu) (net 25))
 (segment (start 129.54 62.865) (end 130.81 61.595) (width 0.4064) (layer B.Cu) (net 25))
 (segment (start 129.54 76.2) (end 129.54 62.865) (width 0.4064) (layer B.Cu) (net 25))
 (segment (start 128.27 77.47) (end 129.54 76.2) (width 0.4064) (layer B.Cu) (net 25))
 (segment (start 134.62 105.41) (end 133.35 104.14) (width 0.4064) (layer B.Cu) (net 15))
 (segment (start 133.35 104.14) (end 128.35 104.14) (width 0.4064) (layer B.Cu) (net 15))
 (segment (start 128.35 104.14) (end 128.27 104.06) (width 0.4064) (layer B.Cu) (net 15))
 (segment (start 134.62 107.95) (end 133.35 106.68) (width 0.4064) (layer B.Cu) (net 16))
 (segment (start 133.35 106.68) (end 128.39 106.68) (width 0.4064) (layer B.Cu) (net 16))
 (segment (start 128.39 106.68) (end 128.27 106.56) (width 0.4064) (layer B.Cu) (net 16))
 (segment (start 128.27 93.82) (end 127.16 93.82) (width 0.4064) (layer F.Cu) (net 17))
 (segment (start 126.84 109.06) (end 128.27 109.06) (width 0.4064) (layer F.Cu) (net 17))
 (segment (start 125.73 107.95) (end 126.84 109.06) (width 0.4064) (layer F.Cu) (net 17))
 (segment (start 125.73 95.25) (end 125.73 107.95) (width 0.4064) (layer F.Cu) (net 17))
 (segment (start 127.16 93.82) (end 125.73 95.25) (width 0.4064) (layer F.Cu) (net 17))
 (segment (start 134.62 63.5) (end 134.62 64.77) (width 0.4064) (layer F.Cu) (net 17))
 (segment (start 127.475 93.82) (end 128.27 93.82) (width 0.4064) (layer F.Cu) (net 17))
 (segment (start 125.73 92.075) (end 127.475 93.82) (width 0.4064) (layer F.Cu) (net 17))
 (segment (start 125.73 83.185) (end 125.73 92.075) (width 0.4064) (layer F.Cu) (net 17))
 (segment (start 130.175 78.74) (end 125.73 83.185) (width 0.4064) (layer F.Cu) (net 17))
 (segment (start 130.175 69.215) (end 130.175 78.74) (width 0.4064) (layer F.Cu) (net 17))
 (segment (start 134.62 64.77) (end 130.175 69.215) (width 0.4064) (layer F.Cu) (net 17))
 (segment (start 134.62 92.71) (end 133.35 91.44) (width 0.4064) (layer B.Cu) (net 10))
 (segment (start 127 89.535) (end 127.715 88.82) (width 0.4064) (layer B.Cu) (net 10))
 (segment (start 127 92.075) (end 127 89.535) (width 0.4064) (layer B.Cu) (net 10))
 (segment (start 127.635 92.71) (end 127 92.075) (width 0.4064) (layer B.Cu) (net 10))
 (segment (start 129.54 92.71) (end 127.635 92.71) (width 0.4064) (layer B.Cu) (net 10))
 (segment (start 130.81 91.44) (end 129.54 92.71) (width 0.4064) (layer B.Cu) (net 10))
 (segment (start 133.35 91.44) (end 130.81 91.44) (width 0.4064) (layer B.Cu) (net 10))
 (segment (start 127.715 88.82) (end 128.27 88.82) (width 0.4064) (layer B.Cu) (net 10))
 (segment (start 134.62 90.17) (end 133.35 88.9) (width 0.4064) (layer B.Cu) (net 9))
 (segment (start 130.81 88.9) (end 128.39 91.32) (width 0.4064) (layer B.Cu) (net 9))
 (segment (start 133.35 88.9) (end 130.81 88.9) (width 0.4064) (layer B.Cu) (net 9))
 (segment (start 128.39 91.32) (end 128.27 91.32) (width 0.4064) (layer B.Cu) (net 9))
 (segment (start 134.366 112.014) (end 135.128 112.014) (width 0.4064) (layer B.Cu) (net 21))
 (segment (start 133.35 113.03) (end 134.366 112.014) (width 0.4064) (layer B.Cu) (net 21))
 (segment (start 133.35 115.062) (end 133.35 113.03) (width 0.4064) (layer B.Cu) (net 21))
 (segment (start 132.207 116.205) (end 133.35 115.062) (width 0.4064) (layer B.Cu) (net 21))
 (segment (start 142.748 85.09) (end 144.78 85.09) (width 0.4064) (layer B.Cu) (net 21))
 (segment (start 137.668 90.17) (end 142.748 85.09) (width 0.4064) (layer B.Cu) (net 21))
 (segment (start 137.668 109.474) (end 137.668 90.17) (width 0.4064) (layer B.Cu) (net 21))
 (segment (start 135.128 112.014) (end 137.668 109.474) (width 0.4064) (layer B.Cu) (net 21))
 (segment (start 132.08 116.205) (end 132.207 116.205) (width 0.4064) (layer B.Cu) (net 21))
 (segment (start 134.874 110.236) (end 132.588 112.522) (width 0.4064) (layer B.Cu) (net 22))
 (segment (start 136.906 86.106) (end 136.906 108.966) (width 0.4064) (layer B.Cu) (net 22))
 (segment (start 136.906 108.966) (end 135.636 110.236) (width 0.4064) (layer B.Cu) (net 22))
 (segment (start 135.636 110.236) (end 134.874 110.236) (width 0.4064) (layer B.Cu) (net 22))
 (segment (start 144.78 82.55) (end 143.002 82.55) (width 0.4064) (layer B.Cu) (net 22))
 (segment (start 140.97 82.042) (end 137.414 85.598) (width 0.4064) (layer B.Cu) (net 22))
 (segment (start 142.494 82.042) (end 140.97 82.042) (width 0.4064) (layer B.Cu) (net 22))
 (segment (start 143.002 82.55) (end 142.494 82.042) (width 0.4064) (layer B.Cu) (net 22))
 (segment (start 137.414 85.598) (end 136.906 86.106) (width 0.4064) (layer B.Cu) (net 22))
 (segment (start 132.588 112.522) (end 132.588 113.157) (width 0.4064) (layer B.Cu) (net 22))
 (segment (start 132.588 113.157) (end 132.08 113.665) (width 0.4064) (layer B.Cu) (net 22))
 (segment (start 137.16 116.205) (end 137.795 116.205) (width 0.4064) (layer B.Cu) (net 19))
 (segment (start 137.795 116.205) (end 139.7 114.3) (width 0.4064) (layer B.Cu) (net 19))
 (segment (start 139.7 114.3) (end 139.7 97.79) (width 0.4064) (layer B.Cu) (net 19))
 (segment (start 139.7 97.79) (end 140.97 96.52) (width 0.4064) (layer B.Cu) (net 19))
 (segment (start 140.97 96.52) (end 143.51 96.52) (width 0.4064) (layer B.Cu) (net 19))
 (segment (start 143.51 96.52) (end 144.78 95.25) (width 0.4064) (layer B.Cu) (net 19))
 (segment (start 144.78 92.71) (end 143.51 93.98) (width 0.4064) (layer B.Cu) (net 20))
 (segment (start 138.43 112.395) (end 137.16 113.665) (width 0.4064) (layer B.Cu) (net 20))
 (segment (start 138.43 96.52) (end 138.43 112.395) (width 0.4064) (layer B.Cu) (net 20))
 (segment (start 140.97 93.98) (end 138.43 96.52) (width 0.4064) (layer B.Cu) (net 20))
 (segment (start 143.51 93.98) (end 140.97 93.98) (width 0.4064) (layer B.Cu) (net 20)))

